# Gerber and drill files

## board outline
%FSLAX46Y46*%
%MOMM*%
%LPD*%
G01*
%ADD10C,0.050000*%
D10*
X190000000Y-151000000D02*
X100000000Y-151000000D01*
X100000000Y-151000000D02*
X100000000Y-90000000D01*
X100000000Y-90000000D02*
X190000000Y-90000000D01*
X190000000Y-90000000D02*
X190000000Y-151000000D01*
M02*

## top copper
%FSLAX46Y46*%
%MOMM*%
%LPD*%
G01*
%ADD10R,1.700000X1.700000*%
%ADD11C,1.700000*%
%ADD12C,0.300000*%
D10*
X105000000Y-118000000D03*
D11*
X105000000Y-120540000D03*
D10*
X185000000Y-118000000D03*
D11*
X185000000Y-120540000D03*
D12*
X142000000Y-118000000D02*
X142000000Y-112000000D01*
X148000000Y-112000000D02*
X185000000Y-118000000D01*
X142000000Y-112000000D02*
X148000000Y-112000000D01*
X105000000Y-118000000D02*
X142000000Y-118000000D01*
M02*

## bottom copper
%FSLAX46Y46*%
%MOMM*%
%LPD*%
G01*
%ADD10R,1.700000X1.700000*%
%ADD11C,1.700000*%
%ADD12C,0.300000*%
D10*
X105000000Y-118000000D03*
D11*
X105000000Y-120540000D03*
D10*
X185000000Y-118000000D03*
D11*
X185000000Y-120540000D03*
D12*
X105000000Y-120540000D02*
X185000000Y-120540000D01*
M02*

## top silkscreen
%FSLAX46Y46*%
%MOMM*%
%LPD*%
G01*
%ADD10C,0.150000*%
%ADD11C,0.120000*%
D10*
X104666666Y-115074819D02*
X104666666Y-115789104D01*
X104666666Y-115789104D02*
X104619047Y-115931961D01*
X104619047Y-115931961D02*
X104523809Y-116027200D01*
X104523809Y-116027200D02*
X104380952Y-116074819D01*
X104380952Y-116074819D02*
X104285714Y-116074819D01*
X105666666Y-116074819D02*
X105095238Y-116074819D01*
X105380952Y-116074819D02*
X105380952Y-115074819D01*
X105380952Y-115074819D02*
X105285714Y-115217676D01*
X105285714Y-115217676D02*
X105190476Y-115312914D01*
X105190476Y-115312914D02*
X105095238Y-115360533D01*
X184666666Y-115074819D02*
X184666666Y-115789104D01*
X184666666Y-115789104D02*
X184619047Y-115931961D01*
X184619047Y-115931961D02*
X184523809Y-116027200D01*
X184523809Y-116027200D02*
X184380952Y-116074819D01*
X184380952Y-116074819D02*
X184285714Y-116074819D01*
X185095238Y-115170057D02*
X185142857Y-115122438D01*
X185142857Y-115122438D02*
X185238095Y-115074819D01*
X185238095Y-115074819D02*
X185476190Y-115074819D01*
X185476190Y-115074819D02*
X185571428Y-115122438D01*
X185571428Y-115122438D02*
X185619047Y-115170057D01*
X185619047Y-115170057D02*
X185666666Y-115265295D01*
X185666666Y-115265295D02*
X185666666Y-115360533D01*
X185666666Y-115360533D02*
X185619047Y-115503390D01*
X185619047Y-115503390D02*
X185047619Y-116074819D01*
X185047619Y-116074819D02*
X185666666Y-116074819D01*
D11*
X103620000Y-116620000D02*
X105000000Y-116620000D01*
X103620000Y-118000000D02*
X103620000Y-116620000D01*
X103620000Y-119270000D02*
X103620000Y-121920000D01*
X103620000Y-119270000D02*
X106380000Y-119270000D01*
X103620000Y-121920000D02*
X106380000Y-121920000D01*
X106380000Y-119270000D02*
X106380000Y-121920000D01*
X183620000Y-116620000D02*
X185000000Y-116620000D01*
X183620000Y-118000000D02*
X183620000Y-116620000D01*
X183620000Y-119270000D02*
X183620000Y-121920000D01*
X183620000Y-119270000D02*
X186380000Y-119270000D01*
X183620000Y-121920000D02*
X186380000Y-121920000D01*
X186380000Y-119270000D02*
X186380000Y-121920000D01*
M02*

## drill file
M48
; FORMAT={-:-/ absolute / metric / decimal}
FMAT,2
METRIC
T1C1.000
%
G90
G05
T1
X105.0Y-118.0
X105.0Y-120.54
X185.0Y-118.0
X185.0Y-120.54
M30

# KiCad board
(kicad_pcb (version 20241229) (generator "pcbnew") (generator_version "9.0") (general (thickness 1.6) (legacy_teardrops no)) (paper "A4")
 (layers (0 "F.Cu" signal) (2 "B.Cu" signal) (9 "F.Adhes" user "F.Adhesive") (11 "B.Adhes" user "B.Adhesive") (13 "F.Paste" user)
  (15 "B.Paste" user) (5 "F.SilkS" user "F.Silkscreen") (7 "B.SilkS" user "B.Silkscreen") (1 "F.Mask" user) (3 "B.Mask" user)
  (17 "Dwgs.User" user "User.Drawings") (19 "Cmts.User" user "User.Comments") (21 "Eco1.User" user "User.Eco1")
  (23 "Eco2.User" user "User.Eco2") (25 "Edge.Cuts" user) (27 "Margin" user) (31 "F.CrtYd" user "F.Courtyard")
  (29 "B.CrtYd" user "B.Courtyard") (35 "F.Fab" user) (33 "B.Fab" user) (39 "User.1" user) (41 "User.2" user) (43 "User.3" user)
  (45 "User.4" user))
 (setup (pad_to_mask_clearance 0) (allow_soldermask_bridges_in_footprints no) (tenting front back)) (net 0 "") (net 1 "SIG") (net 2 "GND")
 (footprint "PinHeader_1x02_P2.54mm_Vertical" (layer "F.Cu") (at 105 118)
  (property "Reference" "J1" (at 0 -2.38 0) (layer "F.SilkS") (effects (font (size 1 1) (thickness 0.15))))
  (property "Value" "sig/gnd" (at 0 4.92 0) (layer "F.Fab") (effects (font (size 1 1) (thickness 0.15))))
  (fp_line (start -1.38 -1.38) (end 0 -1.38) (stroke (width 0.12) (type solid)) (layer "F.SilkS"))
  (fp_line (start -1.38 0) (end -1.38 -1.38) (stroke (width 0.12) (type solid)) (layer "F.SilkS"))
  (fp_line (start -1.38 1.27) (end -1.38 3.92) (stroke (width 0.12) (type solid)) (layer "F.SilkS"))
  (fp_line (start -1.38 1.27) (end 1.38 1.27) (stroke (width 0.12) (type solid)) (layer "F.SilkS"))
  (fp_line (start -1.38 3.92) (end 1.38 3.92) (stroke (width 0.12) (type solid)) (layer "F.SilkS"))
  (fp_line (start 1.38 1.27) (end 1.38 3.92) (stroke (width 0.12) (type solid)) (layer "F.SilkS"))
  (pad "1" thru_hole rect (at 0 0) (size 1.7 1.7) (drill 1) (layers "*.Cu" "*.Mask") (remove_unused_layers no) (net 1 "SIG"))
  (pad "2" thru_hole circle (at 0 2.54) (size 1.7 1.7) (drill 1) (layers "*.Cu" "*.Mask") (remove_unused_layers no) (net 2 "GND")))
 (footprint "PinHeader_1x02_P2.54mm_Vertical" (layer "F.Cu") (at 185 118)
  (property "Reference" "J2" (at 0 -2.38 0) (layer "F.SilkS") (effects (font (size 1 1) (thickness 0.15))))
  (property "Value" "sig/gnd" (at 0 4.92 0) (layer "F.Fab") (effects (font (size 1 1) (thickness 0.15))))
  (fp_line (start -1.38 -1.38) (end 0 -1.38) (stroke (width 0.12) (type solid)) (layer "F.SilkS"))
  (fp_line (start -1.38 0) (end -1.38 -1.38) (stroke (width 0.12) (type solid)) (layer "F.SilkS"))
  (fp_line (start -1.38 1.27) (end -1.38 3.92) (stroke (width 0.12) (type solid)) (layer "F.SilkS"))
  (fp_line (start -1.38 1.27) (end 1.38 1.27) (stroke (width 0.12) (type solid)) (layer "F.SilkS"))
  (fp_line (start -1.38 3.92) (end 1.38 3.92) (stroke (width 0.12) (type solid)) (layer "F.SilkS"))
  (fp_line (start 1.38 1.27) (end 1.38 3.92) (stroke (width 0.12) (type solid)) (layer "F.SilkS"))
  (pad "1" thru_hole rect (at 0 0) (size 1.7 1.7) (drill 1) (layers "*.Cu" "*.Mask") (remove_unused_layers no) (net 1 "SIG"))
  (pad "2" thru_hole circle (at 0 2.54) (size 1.7 1.7) (drill 1) (layers "*.Cu" "*.Mask") (remove_unused_layers no) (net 2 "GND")))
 (gr_line (start 190 151) (end 100 151) (stroke (width 0.05) (type default)) (layer "Edge.Cuts"))
 (gr_line (start 100 151) (end 100 90) (stroke (width 0.05) (type default)) (layer "Edge.Cuts"))
 (gr_line (start 100 90) (end 190 90) (stroke (width 0.05) (type default)) (layer "Edge.Cuts"))
 (gr_line (start 190 90) (end 190 151) (stroke (width 0.05) (type default)) (layer "Edge.Cuts"))
 (segment (start 142 118) (end 142 112) (width 0.3) (layer "F.Cu") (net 1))
 (segment (start 148 112) (end 185 118) (width 0.3) (layer "F.Cu") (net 1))
 (segment (start 142 112) (end 148 112) (width 0.3) (layer "F.Cu") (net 1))
 (segment (start 105 118) (end 142 118) (width 0.3) (layer "F.Cu") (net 1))
 (segment (start 105 120.54) (end 185 120.54) (width 0.3) (layer "B.Cu") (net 2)))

